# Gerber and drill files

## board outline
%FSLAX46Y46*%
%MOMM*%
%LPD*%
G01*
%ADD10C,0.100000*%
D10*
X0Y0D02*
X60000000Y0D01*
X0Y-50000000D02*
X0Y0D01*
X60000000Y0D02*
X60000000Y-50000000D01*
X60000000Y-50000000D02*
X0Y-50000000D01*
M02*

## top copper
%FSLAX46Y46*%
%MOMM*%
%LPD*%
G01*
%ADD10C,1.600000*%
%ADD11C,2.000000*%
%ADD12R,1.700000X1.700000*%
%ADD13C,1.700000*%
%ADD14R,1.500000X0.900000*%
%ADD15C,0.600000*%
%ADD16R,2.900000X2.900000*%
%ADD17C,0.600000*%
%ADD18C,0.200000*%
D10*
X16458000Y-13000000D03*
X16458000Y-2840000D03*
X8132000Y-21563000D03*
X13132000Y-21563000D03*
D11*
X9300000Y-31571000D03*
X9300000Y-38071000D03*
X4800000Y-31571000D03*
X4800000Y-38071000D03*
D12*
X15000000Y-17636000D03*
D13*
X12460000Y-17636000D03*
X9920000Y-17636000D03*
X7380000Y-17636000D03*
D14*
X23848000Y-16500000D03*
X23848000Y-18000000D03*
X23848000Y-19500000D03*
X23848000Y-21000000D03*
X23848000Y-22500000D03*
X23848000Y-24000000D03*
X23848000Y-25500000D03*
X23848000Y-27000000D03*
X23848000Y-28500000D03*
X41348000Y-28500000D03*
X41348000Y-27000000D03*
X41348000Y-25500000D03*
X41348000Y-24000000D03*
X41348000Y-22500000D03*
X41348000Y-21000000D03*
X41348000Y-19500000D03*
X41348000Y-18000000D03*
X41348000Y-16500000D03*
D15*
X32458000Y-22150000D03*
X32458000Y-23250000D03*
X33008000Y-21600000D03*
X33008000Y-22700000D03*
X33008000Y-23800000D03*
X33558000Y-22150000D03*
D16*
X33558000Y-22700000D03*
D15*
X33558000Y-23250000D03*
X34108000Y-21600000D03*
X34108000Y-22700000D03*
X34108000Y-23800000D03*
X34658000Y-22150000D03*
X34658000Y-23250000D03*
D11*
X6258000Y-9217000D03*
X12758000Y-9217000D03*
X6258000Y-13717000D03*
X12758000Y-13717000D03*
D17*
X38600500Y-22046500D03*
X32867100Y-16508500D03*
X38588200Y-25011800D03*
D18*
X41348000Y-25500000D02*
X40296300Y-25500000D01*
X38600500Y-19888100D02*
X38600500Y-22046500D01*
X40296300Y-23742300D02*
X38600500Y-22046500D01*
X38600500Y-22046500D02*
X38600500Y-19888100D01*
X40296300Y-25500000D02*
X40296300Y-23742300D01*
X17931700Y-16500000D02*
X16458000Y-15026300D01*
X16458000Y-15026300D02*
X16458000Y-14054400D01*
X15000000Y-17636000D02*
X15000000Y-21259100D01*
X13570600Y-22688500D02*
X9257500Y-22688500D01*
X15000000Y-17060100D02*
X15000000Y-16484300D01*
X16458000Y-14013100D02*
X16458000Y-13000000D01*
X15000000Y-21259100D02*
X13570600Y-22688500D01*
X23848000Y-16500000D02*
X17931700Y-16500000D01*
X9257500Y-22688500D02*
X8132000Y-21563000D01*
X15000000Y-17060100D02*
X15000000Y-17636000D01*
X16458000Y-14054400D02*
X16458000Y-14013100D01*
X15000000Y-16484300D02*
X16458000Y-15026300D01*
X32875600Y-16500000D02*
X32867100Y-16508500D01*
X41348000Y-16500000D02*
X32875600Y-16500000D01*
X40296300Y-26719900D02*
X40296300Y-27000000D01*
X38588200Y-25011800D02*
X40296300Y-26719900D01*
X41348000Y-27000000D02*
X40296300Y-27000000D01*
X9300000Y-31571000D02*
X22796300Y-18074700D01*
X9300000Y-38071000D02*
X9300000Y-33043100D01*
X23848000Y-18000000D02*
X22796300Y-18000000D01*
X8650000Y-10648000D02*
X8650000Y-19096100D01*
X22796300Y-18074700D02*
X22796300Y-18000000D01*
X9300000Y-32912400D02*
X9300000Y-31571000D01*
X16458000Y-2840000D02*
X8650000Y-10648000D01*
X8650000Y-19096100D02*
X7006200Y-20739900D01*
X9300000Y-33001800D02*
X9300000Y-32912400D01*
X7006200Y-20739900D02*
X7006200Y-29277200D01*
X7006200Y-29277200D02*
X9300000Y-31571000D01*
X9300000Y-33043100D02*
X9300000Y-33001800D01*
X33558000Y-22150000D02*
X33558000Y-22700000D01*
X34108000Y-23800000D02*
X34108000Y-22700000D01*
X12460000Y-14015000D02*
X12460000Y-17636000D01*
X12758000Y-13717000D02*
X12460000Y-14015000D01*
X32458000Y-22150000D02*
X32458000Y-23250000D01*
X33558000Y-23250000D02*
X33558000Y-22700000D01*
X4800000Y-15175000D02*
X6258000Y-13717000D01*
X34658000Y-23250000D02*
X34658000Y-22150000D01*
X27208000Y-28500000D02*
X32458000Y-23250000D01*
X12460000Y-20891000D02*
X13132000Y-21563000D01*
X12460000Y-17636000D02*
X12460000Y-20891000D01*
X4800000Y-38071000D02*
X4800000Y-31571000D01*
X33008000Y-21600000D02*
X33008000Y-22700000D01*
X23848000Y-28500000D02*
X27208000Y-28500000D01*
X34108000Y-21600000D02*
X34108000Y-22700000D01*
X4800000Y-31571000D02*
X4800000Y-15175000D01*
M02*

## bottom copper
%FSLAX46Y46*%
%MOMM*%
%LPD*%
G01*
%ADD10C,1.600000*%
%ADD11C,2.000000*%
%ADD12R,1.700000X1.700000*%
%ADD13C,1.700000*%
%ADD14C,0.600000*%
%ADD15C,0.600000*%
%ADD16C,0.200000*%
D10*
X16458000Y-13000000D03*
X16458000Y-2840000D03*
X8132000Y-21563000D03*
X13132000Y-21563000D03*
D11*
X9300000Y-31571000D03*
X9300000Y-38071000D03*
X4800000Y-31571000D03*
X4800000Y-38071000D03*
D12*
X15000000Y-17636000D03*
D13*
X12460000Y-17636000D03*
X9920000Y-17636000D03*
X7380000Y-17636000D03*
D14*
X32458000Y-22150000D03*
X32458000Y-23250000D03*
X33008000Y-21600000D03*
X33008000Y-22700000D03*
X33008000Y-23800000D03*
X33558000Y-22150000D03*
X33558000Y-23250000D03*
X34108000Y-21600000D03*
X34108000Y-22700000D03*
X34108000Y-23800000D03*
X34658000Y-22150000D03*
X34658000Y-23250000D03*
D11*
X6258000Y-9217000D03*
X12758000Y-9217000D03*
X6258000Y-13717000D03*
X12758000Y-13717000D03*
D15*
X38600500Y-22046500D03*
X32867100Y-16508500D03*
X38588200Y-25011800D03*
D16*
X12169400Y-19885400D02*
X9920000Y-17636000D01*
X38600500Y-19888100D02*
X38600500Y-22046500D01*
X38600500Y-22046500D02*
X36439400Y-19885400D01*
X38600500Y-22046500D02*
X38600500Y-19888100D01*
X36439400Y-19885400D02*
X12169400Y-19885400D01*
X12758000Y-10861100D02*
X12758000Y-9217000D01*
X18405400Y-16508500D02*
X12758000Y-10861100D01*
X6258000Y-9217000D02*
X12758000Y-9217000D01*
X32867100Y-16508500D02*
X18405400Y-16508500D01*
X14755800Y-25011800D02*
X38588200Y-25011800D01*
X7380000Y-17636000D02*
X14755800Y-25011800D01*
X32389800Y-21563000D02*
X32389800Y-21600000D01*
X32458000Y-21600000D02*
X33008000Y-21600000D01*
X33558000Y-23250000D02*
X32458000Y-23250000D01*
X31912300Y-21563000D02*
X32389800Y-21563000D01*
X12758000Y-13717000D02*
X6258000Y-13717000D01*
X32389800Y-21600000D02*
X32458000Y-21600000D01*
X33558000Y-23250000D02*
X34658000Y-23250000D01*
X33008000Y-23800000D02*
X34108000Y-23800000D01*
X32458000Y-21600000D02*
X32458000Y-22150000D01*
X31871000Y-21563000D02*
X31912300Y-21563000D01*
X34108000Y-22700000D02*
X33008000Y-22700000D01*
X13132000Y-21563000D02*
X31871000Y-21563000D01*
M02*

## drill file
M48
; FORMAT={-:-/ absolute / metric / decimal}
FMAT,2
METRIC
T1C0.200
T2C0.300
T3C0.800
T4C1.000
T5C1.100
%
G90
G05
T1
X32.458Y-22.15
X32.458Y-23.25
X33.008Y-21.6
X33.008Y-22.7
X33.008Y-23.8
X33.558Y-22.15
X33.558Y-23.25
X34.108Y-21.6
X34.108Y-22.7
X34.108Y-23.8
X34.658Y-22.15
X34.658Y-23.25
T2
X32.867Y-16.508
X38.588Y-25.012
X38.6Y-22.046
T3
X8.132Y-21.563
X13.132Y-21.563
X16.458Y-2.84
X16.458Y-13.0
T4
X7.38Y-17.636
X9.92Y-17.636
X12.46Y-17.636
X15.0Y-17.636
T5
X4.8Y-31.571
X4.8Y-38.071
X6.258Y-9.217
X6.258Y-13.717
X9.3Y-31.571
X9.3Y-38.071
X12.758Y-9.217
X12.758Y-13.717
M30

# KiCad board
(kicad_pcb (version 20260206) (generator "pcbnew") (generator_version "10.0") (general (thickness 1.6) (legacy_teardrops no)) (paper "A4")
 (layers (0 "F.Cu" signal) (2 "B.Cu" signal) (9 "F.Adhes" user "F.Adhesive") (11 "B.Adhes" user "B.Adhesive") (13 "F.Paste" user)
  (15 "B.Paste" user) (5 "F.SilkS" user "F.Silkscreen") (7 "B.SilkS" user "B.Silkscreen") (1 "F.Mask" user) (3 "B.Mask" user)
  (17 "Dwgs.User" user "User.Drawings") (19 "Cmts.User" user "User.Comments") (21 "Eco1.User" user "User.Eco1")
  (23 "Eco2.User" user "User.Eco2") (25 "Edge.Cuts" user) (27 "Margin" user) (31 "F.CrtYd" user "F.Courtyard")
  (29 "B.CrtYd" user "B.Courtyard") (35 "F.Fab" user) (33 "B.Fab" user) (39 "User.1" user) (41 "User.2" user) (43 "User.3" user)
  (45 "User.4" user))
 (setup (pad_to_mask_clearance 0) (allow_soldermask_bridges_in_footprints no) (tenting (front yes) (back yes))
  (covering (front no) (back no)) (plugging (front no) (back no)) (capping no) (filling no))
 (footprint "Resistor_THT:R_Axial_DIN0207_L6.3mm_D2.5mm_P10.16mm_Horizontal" (layer "F.Cu") (at 16.458 13 90)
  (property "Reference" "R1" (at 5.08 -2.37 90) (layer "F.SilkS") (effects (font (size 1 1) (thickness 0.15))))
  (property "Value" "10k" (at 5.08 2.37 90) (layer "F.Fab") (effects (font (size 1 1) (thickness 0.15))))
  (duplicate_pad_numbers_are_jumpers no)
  (pad "1" thru_hole circle (at 0 0 90) (size 1.6 1.6) (drill 0.8) (layers "*.Cu" "*.Mask") (remove_unused_layers no) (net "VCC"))
  (pad "2" thru_hole circle (at 10.16 0 90) (size 1.6 1.6) (drill 0.8) (layers "*.Cu" "*.Mask") (remove_unused_layers no) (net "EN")))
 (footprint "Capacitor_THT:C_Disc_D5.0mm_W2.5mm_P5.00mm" (layer "F.Cu") (at 8.132 21.563)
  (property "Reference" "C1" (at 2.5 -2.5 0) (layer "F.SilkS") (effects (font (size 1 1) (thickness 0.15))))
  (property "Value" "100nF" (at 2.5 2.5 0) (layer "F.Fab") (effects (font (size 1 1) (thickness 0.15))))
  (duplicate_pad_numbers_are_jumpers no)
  (pad "1" thru_hole circle (at 0 0) (size 1.6 1.6) (drill 0.8) (layers "*.Cu" "*.Mask") (remove_unused_layers no) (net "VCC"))
  (pad "2" thru_hole circle (at 5 0) (size 1.6 1.6) (drill 0.8) (layers "*.Cu" "*.Mask") (remove_unused_layers no) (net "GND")))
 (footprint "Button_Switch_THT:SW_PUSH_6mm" (layer "F.Cu") (at 9.3 31.571 -90)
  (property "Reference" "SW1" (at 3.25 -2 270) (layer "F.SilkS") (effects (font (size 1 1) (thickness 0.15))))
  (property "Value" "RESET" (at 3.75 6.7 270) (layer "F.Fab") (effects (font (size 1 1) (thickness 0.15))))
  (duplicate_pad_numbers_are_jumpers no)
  (pad "1" thru_hole circle (at 0 0) (size 2 2) (drill 1.1) (layers "*.Cu" "*.Mask") (remove_unused_layers no) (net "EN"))
  (pad "1" thru_hole circle (at 6.5 0) (size 2 2) (drill 1.1) (layers "*.Cu" "*.Mask") (remove_unused_layers no) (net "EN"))
  (pad "2" thru_hole circle (at 0 4.5) (size 2 2) (drill 1.1) (layers "*.Cu" "*.Mask") (remove_unused_layers no) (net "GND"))
  (pad "2" thru_hole circle (at 6.5 4.5) (size 2 2) (drill 1.1) (layers "*.Cu" "*.Mask") (remove_unused_layers no) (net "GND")))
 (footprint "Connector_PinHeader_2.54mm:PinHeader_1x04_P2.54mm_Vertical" (layer "F.Cu") (at 15 17.636 -90)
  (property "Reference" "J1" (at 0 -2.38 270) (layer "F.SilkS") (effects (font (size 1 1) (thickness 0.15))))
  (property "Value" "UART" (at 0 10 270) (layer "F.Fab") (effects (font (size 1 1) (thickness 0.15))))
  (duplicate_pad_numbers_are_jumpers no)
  (pad "1" thru_hole rect (at 0 0 270) (size 1.7 1.7) (drill 1) (layers "*.Cu" "*.Mask") (remove_unused_layers no) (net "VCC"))
  (pad "2" thru_hole circle (at 0 2.54 270) (size 1.7 1.7) (drill 1) (layers "*.Cu" "*.Mask") (remove_unused_layers no) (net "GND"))
  (pad "3" thru_hole circle (at 0 5.08 270) (size 1.7 1.7) (drill 1) (layers "*.Cu" "*.Mask") (remove_unused_layers no) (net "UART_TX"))
  (pad "4" thru_hole circle (at 0 7.62 270) (size 1.7 1.7) (drill 1) (layers "*.Cu" "*.Mask") (remove_unused_layers no) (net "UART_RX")))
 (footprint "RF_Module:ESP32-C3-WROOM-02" (layer "F.Cu") (at 32.598 22.5)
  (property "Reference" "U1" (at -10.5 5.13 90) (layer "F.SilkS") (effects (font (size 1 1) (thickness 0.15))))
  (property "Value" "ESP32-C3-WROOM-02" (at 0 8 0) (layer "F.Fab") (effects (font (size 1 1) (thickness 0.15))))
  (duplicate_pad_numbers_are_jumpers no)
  (pad "" smd rect (at -0.14 -0.9) (size 0.7 0.7) (layers "F.Paste"))
  (pad "" smd rect (at -0.14 0.2) (size 0.7 0.7) (layers "F.Paste"))
  (pad "" smd rect (at -0.14 1.3) (size 0.7 0.7) (layers "F.Paste"))
  (pad "" smd rect (at 0.96 -0.9) (size 0.7 0.7) (layers "F.Paste"))
  (pad "" smd rect (at 0.96 0.2) (size 0.7 0.7) (layers "F.Paste"))
  (pad "" smd rect (at 0.96 1.3) (size 0.7 0.7) (layers "F.Paste"))
  (pad "" smd rect (at 2.06 -0.9) (size 0.7 0.7) (layers "F.Paste"))
  (pad "" smd rect (at 2.06 0.2) (size 0.7 0.7) (layers "F.Paste"))
  (pad "" smd rect (at 2.06 1.3) (size 0.7 0.7) (layers "F.Paste"))
  (pad "1" smd rect (at -8.75 -6) (size 1.5 0.9) (layers "F.Cu" "F.Mask" "F.Paste") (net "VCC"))
  (pad "2" smd rect (at -8.75 -4.5) (size 1.5 0.9) (layers "F.Cu" "F.Mask" "F.Paste") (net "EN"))
  (pad "3" smd rect (at -8.75 -3) (size 1.5 0.9) (layers "F.Cu" "F.Mask" "F.Paste"))
  (pad "4" smd rect (at -8.75 -1.5) (size 1.5 0.9) (layers "F.Cu" "F.Mask" "F.Paste"))
  (pad "5" smd rect (at -8.75 0) (size 1.5 0.9) (layers "F.Cu" "F.Mask" "F.Paste"))
  (pad "6" smd rect (at -8.75 1.5) (size 1.5 0.9) (layers "F.Cu" "F.Mask" "F.Paste"))
  (pad "7" smd rect (at -8.75 3) (size 1.5 0.9) (layers "F.Cu" "F.Mask" "F.Paste"))
  (pad "8" smd rect (at -8.75 4.5) (size 1.5 0.9) (layers "F.Cu" "F.Mask" "F.Paste"))
  (pad "9" smd rect (at -8.75 6) (size 1.5 0.9) (layers "F.Cu" "F.Mask" "F.Paste") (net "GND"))
  (pad "10" smd rect (at 8.75 6) (size 1.5 0.9) (layers "F.Cu" "F.Mask" "F.Paste"))
  (pad "11" smd rect (at 8.75 4.5) (size 1.5 0.9) (layers "F.Cu" "F.Mask" "F.Paste") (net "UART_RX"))
  (pad "12" smd rect (at 8.75 3) (size 1.5 0.9) (layers "F.Cu" "F.Mask" "F.Paste") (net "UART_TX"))
  (pad "13" smd rect (at 8.75 1.5) (size 1.5 0.9) (layers "F.Cu" "F.Mask" "F.Paste"))
  (pad "14" smd rect (at 8.75 0) (size 1.5 0.9) (layers "F.Cu" "F.Mask" "F.Paste"))
  (pad "15" smd rect (at 8.75 -1.5) (size 1.5 0.9) (layers "F.Cu" "F.Mask" "F.Paste"))
  (pad "16" smd rect (at 8.75 -3) (size 1.5 0.9) (layers "F.Cu" "F.Mask" "F.Paste"))
  (pad "17" smd rect (at 8.75 -4.5) (size 1.5 0.9) (layers "F.Cu" "F.Mask" "F.Paste"))
  (pad "18" smd rect (at 8.75 -6) (size 1.5 0.9) (layers "F.Cu" "F.Mask" "F.Paste") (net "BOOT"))
  (pad "19" thru_hole circle (at -0.14 -0.35) (size 0.6 0.6) (drill 0.2) (layers "*.Cu" "F.Mask") (remove_unused_layers no) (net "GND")
   (zone_connect 2))
  (pad "19" thru_hole circle (at -0.14 0.75) (size 0.6 0.6) (drill 0.2) (layers "*.Cu" "F.Mask") (remove_unused_layers no) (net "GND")
   (zone_connect 2))
  (pad "19" thru_hole circle (at 0.41 -0.9) (size 0.6 0.6) (drill 0.2) (layers "*.Cu" "F.Mask") (remove_unused_layers no) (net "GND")
   (zone_connect 2))
  (pad "19" thru_hole circle (at 0.41 0.2) (size 0.6 0.6) (drill 0.2) (layers "*.Cu" "F.Mask") (remove_unused_layers no) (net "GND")
   (zone_connect 2))
  (pad "19" thru_hole circle (at 0.41 1.3) (size 0.6 0.6) (drill 0.2) (layers "*.Cu" "F.Mask") (remove_unused_layers no) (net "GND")
   (zone_connect 2))
  (pad "19" thru_hole circle (at 0.96 -0.35) (size 0.6 0.6) (drill 0.2) (layers "*.Cu" "F.Mask") (remove_unused_layers no) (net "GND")
   (zone_connect 2))
  (pad "19" smd rect (at 0.96 0.2) (size 2.9 2.9) (layers "F.Cu" "F.Mask") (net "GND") (zone_connect 2))
  (pad "19" thru_hole circle (at 0.96 0.75) (size 0.6 0.6) (drill 0.2) (layers "*.Cu" "F.Mask") (remove_unused_layers no) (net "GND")
   (zone_connect 2))
  (pad "19" thru_hole circle (at 1.51 -0.9) (size 0.6 0.6) (drill 0.2) (layers "*.Cu" "F.Mask") (remove_unused_layers no) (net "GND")
   (zone_connect 2))
  (pad "19" thru_hole circle (at 1.51 0.2) (size 0.6 0.6) (drill 0.2) (layers "*.Cu" "F.Mask") (remove_unused_layers no) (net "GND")
   (zone_connect 2))
  (pad "19" thru_hole circle (at 1.51 1.3) (size 0.6 0.6) (drill 0.2) (layers "*.Cu" "F.Mask") (remove_unused_layers no) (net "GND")
   (zone_connect 2))
  (pad "19" thru_hole circle (at 2.06 -0.35) (size 0.6 0.6) (drill 0.2) (layers "*.Cu" "F.Mask") (remove_unused_layers no) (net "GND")
   (zone_connect 2))
  (pad "19" thru_hole circle (at 2.06 0.75) (size 0.6 0.6) (drill 0.2) (layers "*.Cu" "F.Mask") (remove_unused_layers no) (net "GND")
   (zone_connect 2))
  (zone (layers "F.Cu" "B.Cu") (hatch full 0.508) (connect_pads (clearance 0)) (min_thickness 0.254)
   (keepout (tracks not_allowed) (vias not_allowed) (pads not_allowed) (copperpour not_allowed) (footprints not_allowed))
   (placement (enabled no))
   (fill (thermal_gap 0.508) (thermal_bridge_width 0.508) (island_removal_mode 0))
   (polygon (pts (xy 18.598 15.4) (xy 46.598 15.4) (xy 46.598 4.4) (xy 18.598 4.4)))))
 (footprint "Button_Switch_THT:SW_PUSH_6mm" (layer "F.Cu") (at 6.258 9.217)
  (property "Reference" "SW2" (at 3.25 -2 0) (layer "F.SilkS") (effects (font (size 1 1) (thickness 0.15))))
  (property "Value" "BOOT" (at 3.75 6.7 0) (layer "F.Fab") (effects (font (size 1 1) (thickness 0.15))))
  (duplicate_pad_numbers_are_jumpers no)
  (pad "1" thru_hole circle (at 0 0 90) (size 2 2) (drill 1.1) (layers "*.Cu" "*.Mask") (remove_unused_layers no) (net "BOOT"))
  (pad "1" thru_hole circle (at 6.5 0 90) (size 2 2) (drill 1.1) (layers "*.Cu" "*.Mask") (remove_unused_layers no) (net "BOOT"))
  (pad "2" thru_hole circle (at 0 4.5 90) (size 2 2) (drill 1.1) (layers "*.Cu" "*.Mask") (remove_unused_layers no) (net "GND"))
  (pad "2" thru_hole circle (at 6.5 4.5 90) (size 2 2) (drill 1.1) (layers "*.Cu" "*.Mask") (remove_unused_layers no) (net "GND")))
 (gr_line (start 0 0) (end 60 0) (stroke (width 0.1) (type default)) (layer "Edge.Cuts"))
 (gr_line (start 0 50) (end 0 0) (stroke (width 0.1) (type default)) (layer "Edge.Cuts"))
 (gr_line (start 60 0) (end 60 50) (stroke (width 0.1) (type default)) (layer "Edge.Cuts"))
 (gr_line (start 60 50) (end 0 50) (stroke (width 0.1) (type default)) (layer "Edge.Cuts"))
 (segment (start 41.348 25.5) (end 40.2963 25.5) (width 0.2) (layer "F.Cu") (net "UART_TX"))
 (segment (start 38.6005 19.8881) (end 38.6005 22.0465) (width 0.2) (layer "F.Cu") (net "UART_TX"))
 (segment (start 40.2963 23.7423) (end 38.6005 22.0465) (width 0.2) (layer "F.Cu") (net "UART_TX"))
 (segment (start 38.6005 22.0465) (end 38.6005 19.8881) (width 0.2) (layer "F.Cu") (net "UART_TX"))
 (segment (start 40.2963 25.5) (end 40.2963 23.7423) (width 0.2) (layer "F.Cu") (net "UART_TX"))
 (via (at 38.6005 22.0465) (size 0.6) (drill 0.3) (layers "F.Cu" "B.Cu") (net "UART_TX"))
 (segment (start 12.1694 19.8854) (end 9.92 17.636) (width 0.2) (layer "B.Cu") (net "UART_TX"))
 (segment (start 38.6005 19.8881) (end 38.6005 22.0465) (width 0.2) (layer "B.Cu") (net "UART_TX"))
 (segment (start 38.6005 22.0465) (end 36.4394 19.8854) (width 0.2) (layer "B.Cu") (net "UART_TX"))
 (segment (start 38.6005 22.0465) (end 38.6005 19.8881) (width 0.2) (layer "B.Cu") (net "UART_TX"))
 (segment (start 36.4394 19.8854) (end 12.1694 19.8854) (width 0.2) (layer "B.Cu") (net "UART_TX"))
 (segment (start 17.9317 16.5) (end 16.458 15.0263) (width 0.2) (layer "F.Cu") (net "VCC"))
 (segment (start 16.458 15.0263) (end 16.458 14.0544) (width 0.2) (layer "F.Cu") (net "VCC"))
 (segment (start 15 17.636) (end 15 21.2591) (width 0.2) (layer "F.Cu") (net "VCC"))
 (segment (start 13.5706 22.6885) (end 9.2575 22.6885) (width 0.2) (layer "F.Cu") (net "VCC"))
 (segment (start 15 17.0601) (end 15 16.4843) (width 0.2) (layer "F.Cu") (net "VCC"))
 (segment (start 16.458 14.0131) (end 16.458 13) (width 0.2) (layer "F.Cu") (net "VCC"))
 (segment (start 15 21.2591) (end 13.5706 22.6885) (width 0.2) (layer "F.Cu") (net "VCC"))
 (segment (start 23.848 16.5) (end 17.9317 16.5) (width 0.2) (layer "F.Cu") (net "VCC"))
 (segment (start 9.2575 22.6885) (end 8.132 21.563) (width 0.2) (layer "F.Cu") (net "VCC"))
 (segment (start 15 17.0601) (end 15 17.636) (width 0.2) (layer "F.Cu") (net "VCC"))
 (segment (start 16.458 14.0544) (end 16.458 14.0131) (width 0.2) (layer "F.Cu") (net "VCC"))
 (segment (start 15 16.4843) (end 16.458 15.0263) (width 0.2) (layer "F.Cu") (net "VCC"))
 (segment (start 32.8756 16.5) (end 32.8671 16.5085) (width 0.2) (layer "F.Cu") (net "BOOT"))
 (segment (start 41.348 16.5) (end 32.8756 16.5) (width 0.2) (layer "F.Cu") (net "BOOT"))
 (via (at 32.8671 16.5085) (size 0.6) (drill 0.3) (layers "F.Cu" "B.Cu") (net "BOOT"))
 (segment (start 12.758 10.8611) (end 12.758 9.217) (width 0.2) (layer "B.Cu") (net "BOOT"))
 (segment (start 18.4054 16.5085) (end 12.758 10.8611) (width 0.2) (layer "B.Cu") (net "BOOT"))
 (segment (start 6.258 9.217) (end 12.758 9.217) (width 0.2) (layer "B.Cu") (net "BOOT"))
 (segment (start 32.8671 16.5085) (end 18.4054 16.5085) (width 0.2) (layer "B.Cu") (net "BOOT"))
 (segment (start 40.2963 26.7199) (end 40.2963 27) (width 0.2) (layer "F.Cu") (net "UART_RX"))
 (segment (start 38.5882 25.0118) (end 40.2963 26.7199) (width 0.2) (layer "F.Cu") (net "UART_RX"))
 (segment (start 41.348 27) (end 40.2963 27) (width 0.2) (layer "F.Cu") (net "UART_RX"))
 (via (at 38.5882 25.0118) (size 0.6) (drill 0.3) (layers "F.Cu" "B.Cu") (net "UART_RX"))
 (segment (start 14.7558 25.0118) (end 38.5882 25.0118) (width 0.2) (layer "B.Cu") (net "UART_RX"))
 (segment (start 7.38 17.636) (end 14.7558 25.0118) (width 0.2) (layer "B.Cu") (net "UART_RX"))
 (segment (start 9.3 31.571) (end 22.7963 18.0747) (width 0.2) (layer "F.Cu") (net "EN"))
 (segment (start 9.3 38.071) (end 9.3 33.0431) (width 0.2) (layer "F.Cu") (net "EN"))
 (segment (start 23.848 18) (end 22.7963 18) (width 0.2) (layer "F.Cu") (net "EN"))
 (segment (start 8.65 10.648) (end 8.65 19.0961) (width 0.2) (layer "F.Cu") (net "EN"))
 (segment (start 22.7963 18.0747) (end 22.7963 18) (width 0.2) (layer "F.Cu") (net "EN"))
 (segment (start 9.3 32.9124) (end 9.3 31.571) (width 0.2) (layer "F.Cu") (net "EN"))
 (segment (start 16.458 2.84) (end 8.65 10.648) (width 0.2) (layer "F.Cu") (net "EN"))
 (segment (start 8.65 19.0961) (end 7.0062 20.7399) (width 0.2) (layer "F.Cu") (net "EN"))
 (segment (start 9.3 33.0018) (end 9.3 32.9124) (width 0.2) (layer "F.Cu") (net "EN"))
 (segment (start 7.0062 20.7399) (end 7.0062 29.2772) (width 0.2) (layer "F.Cu") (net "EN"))
 (segment (start 7.0062 29.2772) (end 9.3 31.571) (width 0.2) (layer "F.Cu") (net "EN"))
 (segment (start 9.3 33.0431) (end 9.3 33.0018) (width 0.2) (layer "F.Cu") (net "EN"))
 (segment (start 33.558 22.15) (end 33.558 22.7) (width 0.2) (layer "F.Cu") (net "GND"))
 (segment (start 34.108 23.8) (end 34.108 22.7) (width 0.2) (layer "F.Cu") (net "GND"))
 (segment (start 12.46 14.015) (end 12.46 17.636) (width 0.2) (layer "F.Cu") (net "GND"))
 (segment (start 12.758 13.717) (end 12.46 14.015) (width 0.2) (layer "F.Cu") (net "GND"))
 (segment (start 32.458 22.15) (end 32.458 23.25) (width 0.2) (layer "F.Cu") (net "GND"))
 (segment (start 33.558 23.25) (end 33.558 22.7) (width 0.2) (layer "F.Cu") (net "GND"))
 (segment (start 4.8 15.175) (end 6.258 13.717) (width 0.2) (layer "F.Cu") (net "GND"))
 (segment (start 34.658 23.25) (end 34.658 22.15) (width 0.2) (layer "F.Cu") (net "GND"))
 (segment (start 27.208 28.5) (end 32.458 23.25) (width 0.2) (layer "F.Cu") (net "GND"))
 (segment (start 12.46 20.891) (end 13.132 21.563) (width 0.2) (layer "F.Cu") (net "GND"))
 (segment (start 12.46 17.636) (end 12.46 20.891) (width 0.2) (layer "F.Cu") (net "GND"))
 (segment (start 4.8 38.071) (end 4.8 31.571) (width 0.2) (layer "F.Cu") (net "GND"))
 (segment (start 33.008 21.6) (end 33.008 22.7) (width 0.2) (layer "F.Cu") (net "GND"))
 (segment (start 23.848 28.5) (end 27.208 28.5) (width 0.2) (layer "F.Cu") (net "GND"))
 (segment (start 34.108 21.6) (end 34.108 22.7) (width 0.2) (layer "F.Cu") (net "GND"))
 (segment (start 4.8 31.571) (end 4.8 15.175) (width 0.2) (layer "F.Cu") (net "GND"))
 (segment (start 32.3898 21.563) (end 32.3898 21.6) (width 0.2) (layer "B.Cu") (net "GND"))
 (segment (start 32.458 21.6) (end 33.008 21.6) (width 0.2) (layer "B.Cu") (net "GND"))
 (segment (start 33.558 23.25) (end 32.458 23.25) (width 0.2) (layer "B.Cu") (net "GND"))
 (segment (start 31.9123 21.563) (end 32.3898 21.563) (width 0.2) (layer "B.Cu") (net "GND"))
 (segment (start 12.758 13.717) (end 6.258 13.717) (width 0.2) (layer "B.Cu") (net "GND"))
 (segment (start 32.3898 21.6) (end 32.458 21.6) (width 0.2) (layer "B.Cu") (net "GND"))
 (segment (start 33.558 23.25) (end 34.658 23.25) (width 0.2) (layer "B.Cu") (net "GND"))
 (segment (start 33.008 23.8) (end 34.108 23.8) (width 0.2) (layer "B.Cu") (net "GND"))
 (segment (start 32.458 21.6) (end 32.458 22.15) (width 0.2) (layer "B.Cu") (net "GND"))
 (segment (start 31.871 21.563) (end 31.9123 21.563) (width 0.2) (layer "B.Cu") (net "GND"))
 (segment (start 34.108 22.7) (end 33.008 22.7) (width 0.2) (layer "B.Cu") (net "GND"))
 (segment (start 13.132 21.563) (end 31.871 21.563) (width 0.2) (layer "B.Cu") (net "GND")))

